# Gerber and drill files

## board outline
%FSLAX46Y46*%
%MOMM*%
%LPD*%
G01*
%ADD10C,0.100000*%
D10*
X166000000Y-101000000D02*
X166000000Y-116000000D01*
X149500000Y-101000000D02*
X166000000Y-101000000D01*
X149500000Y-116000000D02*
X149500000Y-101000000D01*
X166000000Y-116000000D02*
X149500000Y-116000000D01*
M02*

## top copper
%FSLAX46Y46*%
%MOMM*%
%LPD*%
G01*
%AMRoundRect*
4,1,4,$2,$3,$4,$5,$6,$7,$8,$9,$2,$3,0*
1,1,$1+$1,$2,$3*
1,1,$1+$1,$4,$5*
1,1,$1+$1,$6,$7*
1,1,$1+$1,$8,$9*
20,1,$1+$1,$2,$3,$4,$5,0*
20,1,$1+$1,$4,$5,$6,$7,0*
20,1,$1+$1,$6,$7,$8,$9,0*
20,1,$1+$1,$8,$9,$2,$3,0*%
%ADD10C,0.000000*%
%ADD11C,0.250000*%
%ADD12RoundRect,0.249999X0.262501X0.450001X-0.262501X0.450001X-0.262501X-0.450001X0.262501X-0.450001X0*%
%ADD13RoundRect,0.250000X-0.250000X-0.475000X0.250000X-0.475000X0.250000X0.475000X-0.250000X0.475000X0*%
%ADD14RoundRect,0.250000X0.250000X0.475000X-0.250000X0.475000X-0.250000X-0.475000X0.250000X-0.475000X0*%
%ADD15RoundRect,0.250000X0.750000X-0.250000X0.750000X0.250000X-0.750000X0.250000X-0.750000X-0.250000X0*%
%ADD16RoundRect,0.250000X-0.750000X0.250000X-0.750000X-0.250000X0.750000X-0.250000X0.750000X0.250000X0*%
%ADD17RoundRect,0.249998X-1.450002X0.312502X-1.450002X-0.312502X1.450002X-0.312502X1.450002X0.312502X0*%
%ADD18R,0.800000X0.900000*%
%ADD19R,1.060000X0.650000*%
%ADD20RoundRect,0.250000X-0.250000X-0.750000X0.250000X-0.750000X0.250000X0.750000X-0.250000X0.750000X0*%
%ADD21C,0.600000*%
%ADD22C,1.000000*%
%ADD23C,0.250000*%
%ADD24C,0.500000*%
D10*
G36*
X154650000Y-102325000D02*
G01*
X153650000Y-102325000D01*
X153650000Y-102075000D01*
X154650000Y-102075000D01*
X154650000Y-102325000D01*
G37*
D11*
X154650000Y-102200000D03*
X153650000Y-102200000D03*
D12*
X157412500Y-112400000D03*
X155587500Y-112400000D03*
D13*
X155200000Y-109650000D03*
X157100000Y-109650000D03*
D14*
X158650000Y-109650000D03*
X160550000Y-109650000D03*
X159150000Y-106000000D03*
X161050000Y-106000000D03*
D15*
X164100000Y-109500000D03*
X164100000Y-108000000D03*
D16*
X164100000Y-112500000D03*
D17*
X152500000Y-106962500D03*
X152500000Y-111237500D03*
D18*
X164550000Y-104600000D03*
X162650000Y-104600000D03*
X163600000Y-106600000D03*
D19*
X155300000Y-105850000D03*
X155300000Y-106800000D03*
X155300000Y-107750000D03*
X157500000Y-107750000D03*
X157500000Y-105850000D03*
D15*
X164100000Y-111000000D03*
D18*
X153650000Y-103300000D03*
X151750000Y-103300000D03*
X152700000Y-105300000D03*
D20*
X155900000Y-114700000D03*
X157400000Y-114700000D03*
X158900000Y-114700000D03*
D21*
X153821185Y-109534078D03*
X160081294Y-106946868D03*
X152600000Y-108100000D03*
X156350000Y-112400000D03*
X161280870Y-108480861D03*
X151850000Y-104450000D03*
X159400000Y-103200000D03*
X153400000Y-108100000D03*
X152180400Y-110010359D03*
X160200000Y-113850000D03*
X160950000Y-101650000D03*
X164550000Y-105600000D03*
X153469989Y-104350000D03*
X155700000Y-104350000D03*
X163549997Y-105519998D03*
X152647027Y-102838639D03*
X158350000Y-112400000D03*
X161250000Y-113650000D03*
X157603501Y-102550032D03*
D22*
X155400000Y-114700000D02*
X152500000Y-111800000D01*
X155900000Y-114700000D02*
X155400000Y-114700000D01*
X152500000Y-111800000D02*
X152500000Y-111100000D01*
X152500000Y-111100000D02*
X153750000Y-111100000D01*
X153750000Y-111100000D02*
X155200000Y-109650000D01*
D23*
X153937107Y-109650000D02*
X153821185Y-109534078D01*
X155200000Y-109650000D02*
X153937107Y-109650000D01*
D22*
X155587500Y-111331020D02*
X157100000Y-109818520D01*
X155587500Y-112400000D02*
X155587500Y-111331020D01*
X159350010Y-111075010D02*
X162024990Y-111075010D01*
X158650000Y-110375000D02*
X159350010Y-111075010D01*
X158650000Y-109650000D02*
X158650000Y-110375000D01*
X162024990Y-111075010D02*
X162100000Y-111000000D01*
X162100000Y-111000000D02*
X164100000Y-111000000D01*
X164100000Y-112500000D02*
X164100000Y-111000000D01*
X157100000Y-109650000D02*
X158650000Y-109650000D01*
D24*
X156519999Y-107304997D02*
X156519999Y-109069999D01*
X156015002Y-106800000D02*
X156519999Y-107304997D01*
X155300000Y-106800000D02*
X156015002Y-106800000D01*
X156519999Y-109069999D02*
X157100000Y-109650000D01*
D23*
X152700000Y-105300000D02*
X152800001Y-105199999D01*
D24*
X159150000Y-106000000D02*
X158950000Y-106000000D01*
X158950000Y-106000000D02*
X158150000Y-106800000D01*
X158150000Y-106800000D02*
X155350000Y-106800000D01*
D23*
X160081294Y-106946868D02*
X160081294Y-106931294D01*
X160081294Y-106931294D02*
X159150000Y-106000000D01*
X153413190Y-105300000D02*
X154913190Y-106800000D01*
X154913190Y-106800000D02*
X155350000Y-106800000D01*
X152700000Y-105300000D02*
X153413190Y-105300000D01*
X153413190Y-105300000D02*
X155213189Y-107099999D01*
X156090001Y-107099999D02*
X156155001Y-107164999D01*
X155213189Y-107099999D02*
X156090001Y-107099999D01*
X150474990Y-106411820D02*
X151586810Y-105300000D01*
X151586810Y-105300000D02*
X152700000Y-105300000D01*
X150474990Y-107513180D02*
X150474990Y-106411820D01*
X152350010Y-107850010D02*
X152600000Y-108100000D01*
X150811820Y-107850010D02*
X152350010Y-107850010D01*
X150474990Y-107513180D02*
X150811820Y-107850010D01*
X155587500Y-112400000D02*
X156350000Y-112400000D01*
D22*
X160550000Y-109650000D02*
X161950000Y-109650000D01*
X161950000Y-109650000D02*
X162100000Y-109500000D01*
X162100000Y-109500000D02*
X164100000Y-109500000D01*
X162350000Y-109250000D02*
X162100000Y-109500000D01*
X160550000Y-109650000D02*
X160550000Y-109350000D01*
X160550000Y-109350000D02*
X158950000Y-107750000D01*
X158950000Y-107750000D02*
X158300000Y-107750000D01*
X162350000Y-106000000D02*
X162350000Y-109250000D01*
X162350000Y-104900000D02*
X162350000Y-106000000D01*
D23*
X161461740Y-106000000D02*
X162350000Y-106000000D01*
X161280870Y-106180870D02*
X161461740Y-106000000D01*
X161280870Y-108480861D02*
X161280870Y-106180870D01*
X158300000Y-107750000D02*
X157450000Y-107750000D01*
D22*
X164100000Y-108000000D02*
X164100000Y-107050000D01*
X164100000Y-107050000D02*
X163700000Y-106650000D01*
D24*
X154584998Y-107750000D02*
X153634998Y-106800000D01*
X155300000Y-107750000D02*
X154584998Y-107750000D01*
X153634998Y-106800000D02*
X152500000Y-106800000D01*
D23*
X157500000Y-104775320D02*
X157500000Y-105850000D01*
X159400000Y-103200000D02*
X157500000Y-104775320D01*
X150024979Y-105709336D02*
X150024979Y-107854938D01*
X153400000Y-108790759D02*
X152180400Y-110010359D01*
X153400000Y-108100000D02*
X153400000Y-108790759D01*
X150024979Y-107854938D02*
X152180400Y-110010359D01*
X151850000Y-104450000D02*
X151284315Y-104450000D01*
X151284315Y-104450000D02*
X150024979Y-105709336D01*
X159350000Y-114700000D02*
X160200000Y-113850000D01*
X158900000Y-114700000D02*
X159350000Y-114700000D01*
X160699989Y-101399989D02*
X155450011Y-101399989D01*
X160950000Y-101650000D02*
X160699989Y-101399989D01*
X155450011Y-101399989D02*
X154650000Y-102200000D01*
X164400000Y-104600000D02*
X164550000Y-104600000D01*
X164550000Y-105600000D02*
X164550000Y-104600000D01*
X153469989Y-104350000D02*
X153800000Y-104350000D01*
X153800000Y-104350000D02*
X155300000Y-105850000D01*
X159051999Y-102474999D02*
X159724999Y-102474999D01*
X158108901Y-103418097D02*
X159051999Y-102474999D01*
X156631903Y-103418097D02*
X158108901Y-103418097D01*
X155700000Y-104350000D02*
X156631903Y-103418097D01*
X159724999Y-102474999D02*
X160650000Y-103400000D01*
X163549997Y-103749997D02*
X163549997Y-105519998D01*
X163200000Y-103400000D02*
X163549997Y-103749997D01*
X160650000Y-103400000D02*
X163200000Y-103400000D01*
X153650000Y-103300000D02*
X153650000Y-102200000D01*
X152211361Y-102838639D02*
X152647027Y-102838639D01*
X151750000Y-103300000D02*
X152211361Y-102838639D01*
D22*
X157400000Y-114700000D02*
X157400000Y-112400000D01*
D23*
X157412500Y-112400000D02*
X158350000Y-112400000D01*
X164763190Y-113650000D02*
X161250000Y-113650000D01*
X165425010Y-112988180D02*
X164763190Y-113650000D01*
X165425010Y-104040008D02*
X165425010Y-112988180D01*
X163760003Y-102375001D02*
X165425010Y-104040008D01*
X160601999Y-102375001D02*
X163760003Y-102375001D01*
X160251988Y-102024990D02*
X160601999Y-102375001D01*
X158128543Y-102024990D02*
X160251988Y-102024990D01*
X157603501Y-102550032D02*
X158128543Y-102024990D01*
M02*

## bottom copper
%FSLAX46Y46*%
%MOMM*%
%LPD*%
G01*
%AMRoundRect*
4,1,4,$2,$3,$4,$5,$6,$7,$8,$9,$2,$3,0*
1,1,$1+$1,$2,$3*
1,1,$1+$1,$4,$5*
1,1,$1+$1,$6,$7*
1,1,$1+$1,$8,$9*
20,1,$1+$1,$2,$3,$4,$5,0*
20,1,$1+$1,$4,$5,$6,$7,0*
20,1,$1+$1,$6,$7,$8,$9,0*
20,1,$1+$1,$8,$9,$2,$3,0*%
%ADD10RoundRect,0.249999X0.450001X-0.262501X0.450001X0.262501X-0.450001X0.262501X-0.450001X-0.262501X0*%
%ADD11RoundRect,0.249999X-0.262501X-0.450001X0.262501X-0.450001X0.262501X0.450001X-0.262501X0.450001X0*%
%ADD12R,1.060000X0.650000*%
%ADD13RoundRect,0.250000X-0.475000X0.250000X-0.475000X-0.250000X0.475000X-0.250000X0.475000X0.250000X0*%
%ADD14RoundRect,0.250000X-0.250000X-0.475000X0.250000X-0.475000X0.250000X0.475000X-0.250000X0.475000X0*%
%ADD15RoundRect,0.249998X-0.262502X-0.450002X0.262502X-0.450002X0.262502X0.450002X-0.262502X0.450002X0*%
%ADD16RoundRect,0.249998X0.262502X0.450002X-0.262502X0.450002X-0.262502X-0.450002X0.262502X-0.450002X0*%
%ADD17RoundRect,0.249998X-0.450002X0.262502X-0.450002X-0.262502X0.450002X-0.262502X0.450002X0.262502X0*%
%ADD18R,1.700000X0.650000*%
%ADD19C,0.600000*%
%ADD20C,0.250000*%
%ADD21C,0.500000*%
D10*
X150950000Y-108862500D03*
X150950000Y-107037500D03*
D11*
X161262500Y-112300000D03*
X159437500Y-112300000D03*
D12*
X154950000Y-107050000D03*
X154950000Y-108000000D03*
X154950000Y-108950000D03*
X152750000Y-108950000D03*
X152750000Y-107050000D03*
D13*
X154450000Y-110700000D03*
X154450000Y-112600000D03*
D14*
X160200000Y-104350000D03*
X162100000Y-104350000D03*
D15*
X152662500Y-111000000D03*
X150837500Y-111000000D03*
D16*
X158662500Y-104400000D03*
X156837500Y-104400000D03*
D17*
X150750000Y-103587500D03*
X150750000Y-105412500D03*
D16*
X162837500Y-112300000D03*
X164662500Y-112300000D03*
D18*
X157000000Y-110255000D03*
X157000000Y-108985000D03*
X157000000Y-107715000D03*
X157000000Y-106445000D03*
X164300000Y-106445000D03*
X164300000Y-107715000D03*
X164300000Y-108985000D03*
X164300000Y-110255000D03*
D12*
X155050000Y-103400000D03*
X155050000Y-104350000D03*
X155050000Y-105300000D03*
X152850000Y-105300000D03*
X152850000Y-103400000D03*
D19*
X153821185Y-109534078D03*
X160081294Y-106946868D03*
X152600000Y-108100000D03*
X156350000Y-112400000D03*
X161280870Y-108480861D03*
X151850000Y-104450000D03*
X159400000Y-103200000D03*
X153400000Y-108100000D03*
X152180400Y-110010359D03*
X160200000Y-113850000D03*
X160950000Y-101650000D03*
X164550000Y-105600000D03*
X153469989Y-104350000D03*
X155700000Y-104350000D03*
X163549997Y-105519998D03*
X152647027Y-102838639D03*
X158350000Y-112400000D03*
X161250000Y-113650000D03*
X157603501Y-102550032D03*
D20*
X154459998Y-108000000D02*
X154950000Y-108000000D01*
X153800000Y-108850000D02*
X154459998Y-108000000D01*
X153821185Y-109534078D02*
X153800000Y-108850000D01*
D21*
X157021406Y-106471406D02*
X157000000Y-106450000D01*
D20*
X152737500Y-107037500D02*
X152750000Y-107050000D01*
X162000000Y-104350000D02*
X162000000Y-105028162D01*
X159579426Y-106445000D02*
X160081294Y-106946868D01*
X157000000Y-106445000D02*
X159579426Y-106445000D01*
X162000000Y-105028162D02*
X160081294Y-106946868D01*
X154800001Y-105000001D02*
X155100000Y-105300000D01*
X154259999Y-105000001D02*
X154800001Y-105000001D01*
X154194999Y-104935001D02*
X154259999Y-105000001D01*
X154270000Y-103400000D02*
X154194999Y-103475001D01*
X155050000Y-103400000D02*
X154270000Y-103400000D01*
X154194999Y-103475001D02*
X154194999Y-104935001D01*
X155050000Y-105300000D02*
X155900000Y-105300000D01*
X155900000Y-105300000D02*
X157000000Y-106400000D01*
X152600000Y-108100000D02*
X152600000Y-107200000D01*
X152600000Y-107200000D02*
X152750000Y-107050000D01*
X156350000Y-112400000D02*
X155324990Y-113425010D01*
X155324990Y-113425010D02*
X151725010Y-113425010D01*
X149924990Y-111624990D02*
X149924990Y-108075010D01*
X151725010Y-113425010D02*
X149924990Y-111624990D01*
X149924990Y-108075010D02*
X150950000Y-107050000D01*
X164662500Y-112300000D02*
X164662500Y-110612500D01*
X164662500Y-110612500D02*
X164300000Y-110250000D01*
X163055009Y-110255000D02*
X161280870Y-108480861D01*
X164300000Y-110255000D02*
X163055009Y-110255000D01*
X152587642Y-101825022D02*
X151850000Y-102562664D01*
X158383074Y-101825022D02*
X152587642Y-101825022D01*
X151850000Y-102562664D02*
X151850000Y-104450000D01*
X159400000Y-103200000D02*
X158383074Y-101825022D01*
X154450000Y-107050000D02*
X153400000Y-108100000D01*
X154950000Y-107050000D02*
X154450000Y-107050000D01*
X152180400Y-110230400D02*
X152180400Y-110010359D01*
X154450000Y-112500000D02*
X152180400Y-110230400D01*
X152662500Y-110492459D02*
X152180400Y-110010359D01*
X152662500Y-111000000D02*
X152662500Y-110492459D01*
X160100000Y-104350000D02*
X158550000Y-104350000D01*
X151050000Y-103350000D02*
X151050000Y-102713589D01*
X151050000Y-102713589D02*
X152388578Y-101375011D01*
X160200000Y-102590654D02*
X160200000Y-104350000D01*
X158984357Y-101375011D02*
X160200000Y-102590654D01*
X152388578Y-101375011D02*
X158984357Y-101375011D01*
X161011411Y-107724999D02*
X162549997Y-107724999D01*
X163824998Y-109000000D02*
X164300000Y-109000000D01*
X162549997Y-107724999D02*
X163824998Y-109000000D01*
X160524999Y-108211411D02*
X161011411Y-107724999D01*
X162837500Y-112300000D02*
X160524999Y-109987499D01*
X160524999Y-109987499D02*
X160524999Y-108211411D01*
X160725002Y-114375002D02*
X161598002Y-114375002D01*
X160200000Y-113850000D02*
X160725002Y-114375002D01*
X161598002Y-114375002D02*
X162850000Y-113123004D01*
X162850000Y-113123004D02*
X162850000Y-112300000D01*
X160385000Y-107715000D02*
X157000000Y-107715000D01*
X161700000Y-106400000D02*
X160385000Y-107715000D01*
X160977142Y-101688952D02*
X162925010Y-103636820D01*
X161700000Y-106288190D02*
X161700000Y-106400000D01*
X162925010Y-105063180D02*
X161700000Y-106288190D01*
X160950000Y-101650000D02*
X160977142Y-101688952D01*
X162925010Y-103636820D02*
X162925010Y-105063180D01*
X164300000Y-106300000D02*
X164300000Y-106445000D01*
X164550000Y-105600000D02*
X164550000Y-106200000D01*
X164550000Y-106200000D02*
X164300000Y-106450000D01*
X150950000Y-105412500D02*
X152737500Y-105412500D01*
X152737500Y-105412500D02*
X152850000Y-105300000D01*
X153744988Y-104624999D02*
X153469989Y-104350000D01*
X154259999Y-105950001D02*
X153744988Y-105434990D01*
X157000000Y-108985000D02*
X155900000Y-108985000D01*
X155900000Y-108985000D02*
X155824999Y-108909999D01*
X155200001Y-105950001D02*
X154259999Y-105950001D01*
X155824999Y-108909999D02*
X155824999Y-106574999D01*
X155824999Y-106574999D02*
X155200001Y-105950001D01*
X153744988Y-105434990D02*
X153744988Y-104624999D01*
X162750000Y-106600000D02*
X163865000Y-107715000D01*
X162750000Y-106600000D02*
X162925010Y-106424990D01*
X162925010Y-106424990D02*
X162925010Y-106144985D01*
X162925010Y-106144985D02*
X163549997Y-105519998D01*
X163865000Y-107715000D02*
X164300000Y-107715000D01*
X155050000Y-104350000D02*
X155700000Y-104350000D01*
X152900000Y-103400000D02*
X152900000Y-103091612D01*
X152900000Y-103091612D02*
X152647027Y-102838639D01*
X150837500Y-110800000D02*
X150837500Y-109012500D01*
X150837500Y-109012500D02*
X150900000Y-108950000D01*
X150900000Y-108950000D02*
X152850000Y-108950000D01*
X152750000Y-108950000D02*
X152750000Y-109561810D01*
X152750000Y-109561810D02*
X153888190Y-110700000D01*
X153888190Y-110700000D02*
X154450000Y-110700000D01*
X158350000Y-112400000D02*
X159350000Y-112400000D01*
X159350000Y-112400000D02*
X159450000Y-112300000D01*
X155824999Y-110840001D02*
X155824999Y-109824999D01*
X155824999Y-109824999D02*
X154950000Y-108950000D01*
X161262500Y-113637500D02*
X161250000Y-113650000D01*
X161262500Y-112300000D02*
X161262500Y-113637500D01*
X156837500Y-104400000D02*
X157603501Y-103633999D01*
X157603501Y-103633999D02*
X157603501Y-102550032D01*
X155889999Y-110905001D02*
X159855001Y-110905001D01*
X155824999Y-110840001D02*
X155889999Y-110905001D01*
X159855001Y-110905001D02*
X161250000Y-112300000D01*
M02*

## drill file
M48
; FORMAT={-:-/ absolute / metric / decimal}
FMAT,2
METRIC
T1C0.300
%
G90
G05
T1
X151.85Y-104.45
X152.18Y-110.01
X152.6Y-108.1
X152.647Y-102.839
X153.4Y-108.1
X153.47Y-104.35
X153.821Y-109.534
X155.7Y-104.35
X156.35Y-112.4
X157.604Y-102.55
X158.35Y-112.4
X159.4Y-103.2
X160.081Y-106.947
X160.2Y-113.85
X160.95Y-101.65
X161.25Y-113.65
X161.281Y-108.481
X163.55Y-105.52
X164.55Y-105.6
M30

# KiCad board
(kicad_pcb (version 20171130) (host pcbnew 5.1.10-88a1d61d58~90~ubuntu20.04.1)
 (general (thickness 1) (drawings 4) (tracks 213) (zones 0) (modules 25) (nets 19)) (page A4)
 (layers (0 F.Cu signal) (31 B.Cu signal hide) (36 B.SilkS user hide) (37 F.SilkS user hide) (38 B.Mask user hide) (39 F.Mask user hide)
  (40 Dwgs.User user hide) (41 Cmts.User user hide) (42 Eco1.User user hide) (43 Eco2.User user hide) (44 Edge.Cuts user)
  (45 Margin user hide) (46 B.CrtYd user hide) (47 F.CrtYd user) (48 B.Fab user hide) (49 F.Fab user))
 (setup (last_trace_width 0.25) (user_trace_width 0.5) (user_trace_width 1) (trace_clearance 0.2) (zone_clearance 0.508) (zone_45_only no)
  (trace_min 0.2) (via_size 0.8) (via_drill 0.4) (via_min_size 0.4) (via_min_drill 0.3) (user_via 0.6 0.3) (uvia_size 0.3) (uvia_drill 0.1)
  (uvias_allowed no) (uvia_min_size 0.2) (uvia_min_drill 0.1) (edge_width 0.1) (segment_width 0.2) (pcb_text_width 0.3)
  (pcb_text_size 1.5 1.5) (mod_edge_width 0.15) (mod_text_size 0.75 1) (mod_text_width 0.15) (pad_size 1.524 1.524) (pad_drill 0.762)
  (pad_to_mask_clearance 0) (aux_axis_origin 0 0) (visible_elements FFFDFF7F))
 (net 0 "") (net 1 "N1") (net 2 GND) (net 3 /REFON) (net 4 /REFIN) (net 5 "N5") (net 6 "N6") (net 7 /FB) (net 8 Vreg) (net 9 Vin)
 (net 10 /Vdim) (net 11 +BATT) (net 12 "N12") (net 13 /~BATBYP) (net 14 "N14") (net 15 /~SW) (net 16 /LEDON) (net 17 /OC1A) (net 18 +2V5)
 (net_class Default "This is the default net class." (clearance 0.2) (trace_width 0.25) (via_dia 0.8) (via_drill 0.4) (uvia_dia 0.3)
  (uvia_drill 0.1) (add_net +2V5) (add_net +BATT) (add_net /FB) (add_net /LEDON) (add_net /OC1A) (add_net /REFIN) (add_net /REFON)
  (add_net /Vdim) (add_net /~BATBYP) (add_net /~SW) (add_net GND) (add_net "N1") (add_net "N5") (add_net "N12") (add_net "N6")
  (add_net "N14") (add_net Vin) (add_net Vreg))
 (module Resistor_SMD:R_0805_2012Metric (layer B.Cu) (at 150.95 107.95 90)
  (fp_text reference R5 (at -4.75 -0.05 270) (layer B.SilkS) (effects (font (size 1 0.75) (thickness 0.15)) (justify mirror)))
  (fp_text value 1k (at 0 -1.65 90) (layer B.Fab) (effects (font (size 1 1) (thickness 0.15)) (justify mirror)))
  (pad 1 smd roundrect (at -0.9125 0 90) (size 1.025 1.4) (layers B.Cu B.Paste B.Mask) (roundrect_rratio 0.2439014634146341) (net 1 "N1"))
  (pad 2 smd roundrect (at 0.9125 0 90) (size 1.025 1.4) (layers B.Cu B.Paste B.Mask) (roundrect_rratio 0.2439014634146341) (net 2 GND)))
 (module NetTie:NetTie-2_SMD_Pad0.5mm (layer F.Cu) (at 154.15 102.2 180)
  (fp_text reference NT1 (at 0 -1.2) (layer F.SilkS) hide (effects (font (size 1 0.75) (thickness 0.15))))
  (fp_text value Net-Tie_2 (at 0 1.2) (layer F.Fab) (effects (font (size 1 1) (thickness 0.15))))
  (fp_poly (pts (xy -0.5 -0.125) (xy 0.5 -0.125) (xy 0.5 0.125) (xy -0.5 0.125)) (layer F.Cu) (width 0))
  (pad 1 smd circle (at -0.5 0 180) (size 0.25 0.25) (layers F.Cu) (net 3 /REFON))
  (pad 2 smd circle (at 0.5 0 180) (size 0.25 0.25) (layers F.Cu) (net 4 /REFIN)))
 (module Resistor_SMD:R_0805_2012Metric (layer F.Cu) (at 156.5 112.4 180)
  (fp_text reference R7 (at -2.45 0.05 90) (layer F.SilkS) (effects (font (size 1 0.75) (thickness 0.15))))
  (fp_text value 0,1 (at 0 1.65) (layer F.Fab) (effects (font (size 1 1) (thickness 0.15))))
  (pad 1 smd roundrect (at -0.9125 0 180) (size 1.025 1.4) (layers F.Cu F.Paste F.Mask) (roundrect_rratio 0.2439014634146341) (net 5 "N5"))
  (pad 2 smd roundrect (at 0.9125 0 180) (size 1.025 1.4) (layers F.Cu F.Paste F.Mask) (roundrect_rratio 0.2439014634146341) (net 2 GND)))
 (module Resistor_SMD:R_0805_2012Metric (layer B.Cu) (at 160.35 112.3)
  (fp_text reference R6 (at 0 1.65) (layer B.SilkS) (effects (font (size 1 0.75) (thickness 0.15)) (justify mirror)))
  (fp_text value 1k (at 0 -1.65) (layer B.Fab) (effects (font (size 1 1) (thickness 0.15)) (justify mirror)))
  (pad 2 smd roundrect (at 0.9125 0) (size 1.025 1.4) (layers B.Cu B.Paste B.Mask) (roundrect_rratio 0.2439014634146341) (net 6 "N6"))
  (pad 1 smd roundrect (at -0.9125 0) (size 1.025 1.4) (layers B.Cu B.Paste B.Mask) (roundrect_rratio 0.2439014634146341) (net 5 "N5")))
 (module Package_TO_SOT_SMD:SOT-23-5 (layer B.Cu) (at 153.85 108 180)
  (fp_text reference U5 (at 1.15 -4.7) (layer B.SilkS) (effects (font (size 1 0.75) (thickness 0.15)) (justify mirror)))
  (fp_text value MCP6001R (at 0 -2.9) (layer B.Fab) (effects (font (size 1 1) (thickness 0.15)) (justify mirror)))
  (pad 1 smd rect (at -1.1 0.95 180) (size 1.06 0.65) (layers B.Cu B.Paste B.Mask) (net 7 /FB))
  (pad 2 smd rect (at -1.1 0 180) (size 1.06 0.65) (layers B.Cu B.Paste B.Mask) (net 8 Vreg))
  (pad 3 smd rect (at -1.1 -0.95 180) (size 1.06 0.65) (layers B.Cu B.Paste B.Mask) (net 6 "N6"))
  (pad 4 smd rect (at 1.1 -0.95 180) (size 1.06 0.65) (layers B.Cu B.Paste B.Mask) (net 1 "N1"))
  (pad 5 smd rect (at 1.1 0.95 180) (size 1.06 0.65) (layers B.Cu B.Paste B.Mask) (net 2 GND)))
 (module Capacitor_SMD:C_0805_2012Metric (layer F.Cu) (at 156.15 109.65)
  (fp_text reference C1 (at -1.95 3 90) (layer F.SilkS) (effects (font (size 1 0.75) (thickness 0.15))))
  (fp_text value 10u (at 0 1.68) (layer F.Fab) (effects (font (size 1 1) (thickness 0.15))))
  (pad 1 smd roundrect (at -0.95 0) (size 1 1.45) (layers F.Cu F.Paste F.Mask) (roundrect_rratio 0.25) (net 8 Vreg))
  (pad 2 smd roundrect (at 0.95 0) (size 1 1.45) (layers F.Cu F.Paste F.Mask) (roundrect_rratio 0.25) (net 2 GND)))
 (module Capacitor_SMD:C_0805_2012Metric (layer B.Cu) (at 154.45 111.65 270)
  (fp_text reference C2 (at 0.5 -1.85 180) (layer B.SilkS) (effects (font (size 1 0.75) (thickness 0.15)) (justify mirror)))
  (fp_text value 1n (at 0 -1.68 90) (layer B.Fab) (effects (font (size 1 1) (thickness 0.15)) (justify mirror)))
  (pad 1 smd roundrect (at -0.95 0 270) (size 1 1.45) (layers B.Cu B.Paste B.Mask) (roundrect_rratio 0.25) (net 1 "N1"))
  (pad 2 smd roundrect (at 0.95 0 270) (size 1 1.45) (layers B.Cu B.Paste B.Mask) (roundrect_rratio 0.25) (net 7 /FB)))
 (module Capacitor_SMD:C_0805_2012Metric (layer F.Cu) (at 159.6 109.65 180)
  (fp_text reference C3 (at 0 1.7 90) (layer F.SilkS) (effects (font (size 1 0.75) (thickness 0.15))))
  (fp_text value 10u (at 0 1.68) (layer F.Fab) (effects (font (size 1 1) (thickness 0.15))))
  (pad 2 smd roundrect (at 0.95 0 180) (size 1 1.45) (layers F.Cu F.Paste F.Mask) (roundrect_rratio 0.25) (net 2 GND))
  (pad 1 smd roundrect (at -0.95 0 180) (size 1 1.45) (layers F.Cu F.Paste F.Mask) (roundrect_rratio 0.25) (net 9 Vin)))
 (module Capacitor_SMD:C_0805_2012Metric (layer F.Cu) (at 160.1 106 180)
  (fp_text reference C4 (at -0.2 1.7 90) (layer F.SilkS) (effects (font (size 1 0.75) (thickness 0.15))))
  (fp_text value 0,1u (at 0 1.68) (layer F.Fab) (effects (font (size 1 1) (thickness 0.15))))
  (pad 2 smd roundrect (at 0.95 0 180) (size 1 1.45) (layers F.Cu F.Paste F.Mask) (roundrect_rratio 0.25) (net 2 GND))
  (pad 1 smd roundrect (at -0.95 0 180) (size 1 1.45) (layers F.Cu F.Paste F.Mask) (roundrect_rratio 0.25) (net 9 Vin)))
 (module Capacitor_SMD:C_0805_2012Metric (layer B.Cu) (at 161.15 104.35)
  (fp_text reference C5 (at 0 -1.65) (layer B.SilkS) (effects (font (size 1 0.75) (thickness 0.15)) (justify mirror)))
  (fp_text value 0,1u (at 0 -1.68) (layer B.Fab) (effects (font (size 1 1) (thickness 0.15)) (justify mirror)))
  (pad 1 smd roundrect (at -0.95 0) (size 1 1.45) (layers B.Cu B.Paste B.Mask) (roundrect_rratio 0.25) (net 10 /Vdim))
  (pad 2 smd roundrect (at 0.95 0) (size 1 1.45) (layers B.Cu B.Paste B.Mask) (roundrect_rratio 0.25) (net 2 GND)))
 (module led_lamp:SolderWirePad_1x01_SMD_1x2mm (layer F.Cu) (at 164.1 109.5 90)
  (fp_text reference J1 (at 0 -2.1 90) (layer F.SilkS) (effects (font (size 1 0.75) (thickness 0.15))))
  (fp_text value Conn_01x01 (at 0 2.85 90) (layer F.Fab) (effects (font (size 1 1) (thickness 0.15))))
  (pad 1 smd roundrect (at 0 0 90) (size 1 2) (layers F.Cu F.Paste F.Mask) (roundrect_rratio 0.25) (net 9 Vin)))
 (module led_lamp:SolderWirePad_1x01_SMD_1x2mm (layer F.Cu) (at 164.1 108 90)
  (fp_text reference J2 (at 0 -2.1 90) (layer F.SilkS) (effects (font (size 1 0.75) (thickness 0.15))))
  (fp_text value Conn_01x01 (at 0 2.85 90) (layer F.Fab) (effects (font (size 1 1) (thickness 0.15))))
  (pad 1 smd roundrect (at 0 0 90) (size 1 2) (layers F.Cu F.Paste F.Mask) (roundrect_rratio 0.25) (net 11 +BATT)))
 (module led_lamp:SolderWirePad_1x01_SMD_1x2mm (layer F.Cu) (at 164.1 112.5 270)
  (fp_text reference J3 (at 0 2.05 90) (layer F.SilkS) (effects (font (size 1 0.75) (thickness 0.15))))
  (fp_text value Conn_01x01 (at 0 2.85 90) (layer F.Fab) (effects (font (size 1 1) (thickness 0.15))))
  (pad 1 smd roundrect (at 0 0 270) (size 1 2) (layers F.Cu F.Paste F.Mask) (roundrect_rratio 0.25) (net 2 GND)))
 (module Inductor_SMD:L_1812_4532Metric (layer F.Cu) (at 152.5 109.1 270)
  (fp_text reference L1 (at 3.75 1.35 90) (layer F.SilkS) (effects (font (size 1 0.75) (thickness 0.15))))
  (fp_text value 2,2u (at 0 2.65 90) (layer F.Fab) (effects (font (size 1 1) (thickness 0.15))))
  (pad 1 smd roundrect (at -2.1375 0 270) (size 1.125 3.4) (layers F.Cu F.Paste F.Mask) (roundrect_rratio 0.2222204444444444) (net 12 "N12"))
  (pad 2 smd roundrect (at 2.1375 0 270) (size 1.125 3.4) (layers F.Cu F.Paste F.Mask) (roundrect_rratio 0.2222204444444444) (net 8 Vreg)))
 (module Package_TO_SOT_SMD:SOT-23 (layer F.Cu) (at 163.6 105.6 270)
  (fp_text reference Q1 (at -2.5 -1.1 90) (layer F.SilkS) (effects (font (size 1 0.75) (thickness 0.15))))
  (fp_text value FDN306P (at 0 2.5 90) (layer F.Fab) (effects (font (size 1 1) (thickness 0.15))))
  (pad 1 smd rect (at -1 -0.95 270) (size 0.9 0.8) (layers F.Cu F.Paste F.Mask) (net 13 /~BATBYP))
  (pad 2 smd rect (at -1 0.95 270) (size 0.9 0.8) (layers F.Cu F.Paste F.Mask) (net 9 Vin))
  (pad 3 smd rect (at 1 0 270) (size 0.9 0.8) (layers F.Cu F.Paste F.Mask) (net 11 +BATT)))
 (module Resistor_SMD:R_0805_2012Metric (layer B.Cu) (at 151.75 111)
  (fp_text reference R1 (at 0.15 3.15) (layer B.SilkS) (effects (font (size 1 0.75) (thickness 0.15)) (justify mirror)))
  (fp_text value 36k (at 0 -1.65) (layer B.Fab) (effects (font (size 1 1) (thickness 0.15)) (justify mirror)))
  (pad 2 smd roundrect (at 0.9125 0) (size 1.025 1.4) (layers B.Cu B.Paste B.Mask) (roundrect_rratio 0.2439004878048781) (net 7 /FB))
  (pad 1 smd roundrect (at -0.9125 0) (size 1.025 1.4) (layers B.Cu B.Paste B.Mask) (roundrect_rratio 0.2439004878048781) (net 1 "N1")))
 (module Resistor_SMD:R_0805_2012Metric (layer B.Cu) (at 157.75 104.4 180)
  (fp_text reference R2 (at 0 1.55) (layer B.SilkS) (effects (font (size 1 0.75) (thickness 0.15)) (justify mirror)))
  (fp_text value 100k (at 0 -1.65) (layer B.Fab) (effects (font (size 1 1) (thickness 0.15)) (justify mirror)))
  (pad 1 smd roundrect (at -0.9125 0 180) (size 1.025 1.4) (layers B.Cu B.Paste B.Mask) (roundrect_rratio 0.2439004878048781) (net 10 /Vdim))
  (pad 2 smd roundrect (at 0.9125 0 180) (size 1.025 1.4) (layers B.Cu B.Paste B.Mask) (roundrect_rratio 0.2439004878048781) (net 6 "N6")))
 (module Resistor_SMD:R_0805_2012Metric (layer B.Cu) (at 150.75 104.5 270)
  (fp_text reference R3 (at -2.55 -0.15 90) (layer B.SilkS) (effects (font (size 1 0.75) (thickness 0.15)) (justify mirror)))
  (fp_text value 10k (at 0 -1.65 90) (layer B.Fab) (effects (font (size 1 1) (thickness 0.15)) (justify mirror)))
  (pad 1 smd roundrect (at -0.9125 0 270) (size 1.025 1.4) (layers B.Cu B.Paste B.Mask) (roundrect_rratio 0.2439004878048781) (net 10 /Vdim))
  (pad 2 smd roundrect (at 0.9125 0 270) (size 1.025 1.4) (layers B.Cu B.Paste B.Mask) (roundrect_rratio 0.2439004878048781) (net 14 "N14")))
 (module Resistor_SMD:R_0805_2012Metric (layer B.Cu) (at 163.75 112.3 180)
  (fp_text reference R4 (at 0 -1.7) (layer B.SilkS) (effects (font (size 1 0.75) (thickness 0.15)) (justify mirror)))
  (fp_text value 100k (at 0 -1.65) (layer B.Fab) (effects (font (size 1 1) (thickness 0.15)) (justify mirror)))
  (pad 2 smd roundrect (at 0.9125 0 180) (size 1.025 1.4) (layers B.Cu B.Paste B.Mask) (roundrect_rratio 0.2439004878048781) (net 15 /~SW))
  (pad 1 smd roundrect (at -0.9125 0 180) (size 1.025 1.4) (layers B.Cu B.Paste B.Mask) (roundrect_rratio 0.2439004878048781) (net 9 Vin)))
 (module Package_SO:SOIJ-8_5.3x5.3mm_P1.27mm (layer B.Cu) (at 160.65 108.35)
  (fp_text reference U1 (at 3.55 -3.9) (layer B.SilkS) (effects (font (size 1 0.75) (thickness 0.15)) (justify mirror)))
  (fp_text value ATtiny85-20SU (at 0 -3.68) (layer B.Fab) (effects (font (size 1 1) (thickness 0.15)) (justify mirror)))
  (pad 1 smd rect (at -3.65 1.905) (size 1.7 0.65) (layers B.Cu B.Paste B.Mask))
  (pad 2 smd rect (at -3.65 0.635) (size 1.7 0.65) (layers B.Cu B.Paste B.Mask) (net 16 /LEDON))
  (pad 3 smd rect (at -3.65 -0.635) (size 1.7 0.65) (layers B.Cu B.Paste B.Mask) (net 3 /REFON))
  (pad 4 smd rect (at -3.65 -1.905) (size 1.7 0.65) (layers B.Cu B.Paste B.Mask) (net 2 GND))
  (pad 5 smd rect (at 3.65 -1.905) (size 1.7 0.65) (layers B.Cu B.Paste B.Mask) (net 13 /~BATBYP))
  (pad 6 smd rect (at 3.65 -0.635) (size 1.7 0.65) (layers B.Cu B.Paste B.Mask) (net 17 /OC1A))
  (pad 7 smd rect (at 3.65 0.635) (size 1.7 0.65) (layers B.Cu B.Paste B.Mask) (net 15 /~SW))
  (pad 8 smd rect (at 3.65 1.905) (size 1.7 0.65) (layers B.Cu B.Paste B.Mask) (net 9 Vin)))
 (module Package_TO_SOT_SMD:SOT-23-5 (layer F.Cu) (at 156.4 106.8)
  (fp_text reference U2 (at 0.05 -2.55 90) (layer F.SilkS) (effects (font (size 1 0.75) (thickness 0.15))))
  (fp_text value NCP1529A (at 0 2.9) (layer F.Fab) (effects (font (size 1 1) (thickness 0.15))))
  (pad 1 smd rect (at -1.1 -0.95) (size 1.06 0.65) (layers F.Cu F.Paste F.Mask) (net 16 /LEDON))
  (pad 2 smd rect (at -1.1 0) (size 1.06 0.65) (layers F.Cu F.Paste F.Mask) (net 2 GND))
  (pad 3 smd rect (at -1.1 0.95) (size 1.06 0.65) (layers F.Cu F.Paste F.Mask) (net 12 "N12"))
  (pad 4 smd rect (at 1.1 0.95) (size 1.06 0.65) (layers F.Cu F.Paste F.Mask) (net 9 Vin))
  (pad 5 smd rect (at 1.1 -0.95) (size 1.06 0.65) (layers F.Cu F.Paste F.Mask) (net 7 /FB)))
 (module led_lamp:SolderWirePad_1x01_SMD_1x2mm (layer F.Cu) (at 164.1 111 90)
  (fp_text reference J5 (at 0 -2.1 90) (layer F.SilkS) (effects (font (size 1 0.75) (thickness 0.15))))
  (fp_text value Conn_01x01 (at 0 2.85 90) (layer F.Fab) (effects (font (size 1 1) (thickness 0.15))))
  (pad 1 smd roundrect (at 0 0 90) (size 1 2) (layers F.Cu F.Paste F.Mask) (roundrect_rratio 0.25) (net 2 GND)))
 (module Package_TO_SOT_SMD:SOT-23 (layer F.Cu) (at 152.7 104.3 270)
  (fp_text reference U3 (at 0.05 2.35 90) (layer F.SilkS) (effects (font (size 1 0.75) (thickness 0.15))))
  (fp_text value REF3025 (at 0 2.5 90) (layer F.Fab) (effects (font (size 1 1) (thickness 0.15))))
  (pad 1 smd rect (at -1 -0.95 270) (size 0.9 0.8) (layers F.Cu F.Paste F.Mask) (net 4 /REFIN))
  (pad 2 smd rect (at -1 0.95 270) (size 0.9 0.8) (layers F.Cu F.Paste F.Mask) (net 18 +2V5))
  (pad 3 smd rect (at 1 0 270) (size 0.9 0.8) (layers F.Cu F.Paste F.Mask) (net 2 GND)))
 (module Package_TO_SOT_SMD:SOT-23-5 (layer B.Cu) (at 153.95 104.35 180)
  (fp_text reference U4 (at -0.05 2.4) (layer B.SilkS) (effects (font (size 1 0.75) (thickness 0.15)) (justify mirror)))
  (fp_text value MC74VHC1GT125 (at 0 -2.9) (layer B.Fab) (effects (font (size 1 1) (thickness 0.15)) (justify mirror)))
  (pad 1 smd rect (at -1.1 0.95 180) (size 1.06 0.65) (layers B.Cu B.Paste B.Mask) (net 2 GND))
  (pad 2 smd rect (at -1.1 0 180) (size 1.06 0.65) (layers B.Cu B.Paste B.Mask) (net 17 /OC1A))
  (pad 3 smd rect (at -1.1 -0.95 180) (size 1.06 0.65) (layers B.Cu B.Paste B.Mask) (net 2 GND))
  (pad 4 smd rect (at 1.1 -0.95 180) (size 1.06 0.65) (layers B.Cu B.Paste B.Mask) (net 14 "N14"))
  (pad 5 smd rect (at 1.1 0.95 180) (size 1.06 0.65) (layers B.Cu B.Paste B.Mask) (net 18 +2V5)))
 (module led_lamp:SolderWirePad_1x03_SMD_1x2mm (layer F.Cu) (at 155.9 114.7)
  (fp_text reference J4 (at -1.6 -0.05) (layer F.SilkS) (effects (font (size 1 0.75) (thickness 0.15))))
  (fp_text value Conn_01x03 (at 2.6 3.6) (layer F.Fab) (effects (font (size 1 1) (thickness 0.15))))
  (pad 1 smd roundrect (at 0 0) (size 1 2) (layers F.Cu F.Paste F.Mask) (roundrect_rratio 0.25) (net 8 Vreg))
  (pad 2 smd roundrect (at 1.5 0) (size 1 2) (layers F.Cu F.Paste F.Mask) (roundrect_rratio 0.25) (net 5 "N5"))
  (pad 3 smd roundrect (at 3 0) (size 1 2) (layers F.Cu F.Paste F.Mask) (roundrect_rratio 0.25) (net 15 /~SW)))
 (gr_line (start 166 101) (end 166 116) (layer Edge.Cuts) (width 0.1))
 (gr_line (start 149.5 101) (end 166 101) (layer Edge.Cuts) (width 0.1))
 (gr_line (start 149.5 116) (end 149.5 101) (layer Edge.Cuts) (width 0.1))
 (gr_line (start 166 116) (end 149.5 116) (layer Edge.Cuts) (width 0.1))
 (segment (start 155.4 114.7) (end 152.5 111.8) (width 1) (layer F.Cu) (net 8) (status 10))
 (segment (start 155.9 114.7) (end 155.4 114.7) (width 1) (layer F.Cu) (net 8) (status 30))
 (segment (start 152.5 111.8) (end 152.5 111.1) (width 1) (layer F.Cu) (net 8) (status 20))
 (segment (start 152.5 111.1) (end 153.75 111.1) (width 1) (layer F.Cu) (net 8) (status 30))
 (segment (start 153.75 111.1) (end 155.2 109.65) (width 1) (layer F.Cu) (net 8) (status 30))
 (via (at 153.821185 109.534078) (size 0.6) (drill 0.3) (layers F.Cu B.Cu) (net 8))
 (segment (start 153.937107 109.65) (end 153.821185 109.534078) (width 0.25) (layer F.Cu) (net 8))
 (segment (start 155.2 109.65) (end 153.937107 109.65) (width 0.25) (layer F.Cu) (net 8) (status 10))
 (segment (start 154.459998 108) (end 154.95 108) (width 0.25) (layer B.Cu) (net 8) (status 30))
 (segment (start 153.8 108.85) (end 154.459998 108) (width 0.25) (layer B.Cu) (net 8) (status 20))
 (segment (start 153.821185 109.534078) (end 153.8 108.85) (width 0.25) (layer B.Cu) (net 8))
 (segment (start 155.5875 111.33102) (end 157.1 109.81852) (width 1) (layer F.Cu) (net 2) (status 20))
 (segment (start 155.5875 112.4) (end 155.5875 111.33102) (width 1) (layer F.Cu) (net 2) (status 10))
 (segment (start 159.35001 111.07501) (end 162.02499 111.07501) (width 1) (layer F.Cu) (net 2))
 (segment (start 158.65 110.375) (end 159.35001 111.07501) (width 1) (layer F.Cu) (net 2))
 (segment (start 158.65 109.65) (end 158.65 110.375) (width 1) (layer F.Cu) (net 2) (status 10))
 (segment (start 162.02499 111.07501) (end 162.1 111) (width 1) (layer F.Cu) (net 2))
 (segment (start 162.1 111) (end 164.1 111) (width 1) (layer F.Cu) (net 2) (status 20))
 (segment (start 164.1 112.5) (end 164.1 111) (width 1) (layer F.Cu) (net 2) (status 30))
 (segment (start 157.1 109.65) (end 158.65 109.65) (width 1) (layer F.Cu) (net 2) (status 30))
 (segment (start 156.519999 107.304997) (end 156.519999 109.069999) (width 0.5) (layer F.Cu) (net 2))
 (segment (start 156.015002 106.8) (end 156.519999 107.304997) (width 0.5) (layer F.Cu) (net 2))
 (segment (start 155.3 106.8) (end 156.015002 106.8) (width 0.5) (layer F.Cu) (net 2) (status 10))
 (segment (start 156.519999 109.069999) (end 157.1 109.65) (width 0.5) (layer F.Cu) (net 2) (status 20))
 (segment (start 152.7 105.3) (end 152.800001 105.199999) (width 0.25) (layer F.Cu) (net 2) (status 30))
 (segment (start 157.021406 106.471406) (end 157 106.45) (width 0.5) (layer B.Cu) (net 2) (status 30))
 (segment (start 159.15 106) (end 158.95 106) (width 0.5) (layer F.Cu) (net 2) (status 30))
 (segment (start 158.95 106) (end 158.15 106.8) (width 0.5) (layer F.Cu) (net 2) (status 10))
 (segment (start 158.15 106.8) (end 155.35 106.8) (width 0.5) (layer F.Cu) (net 2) (status 20))
 (segment (start 152.7375 107.0375) (end 152.75 107.05) (width 0.25) (layer B.Cu) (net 2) (status 30))
 (segment (start 162 104.35) (end 162 105.028162) (width 0.25) (layer B.Cu) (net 2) (status 30))
 (via (at 160.081294 106.946868) (size 0.6) (drill 0.3) (layers F.Cu B.Cu) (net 2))
 (segment (start 159.579426 106.445) (end 160.081294 106.946868) (width 0.25) (layer B.Cu) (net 2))
 (segment (start 157 106.445) (end 159.579426 106.445) (width 0.25) (layer B.Cu) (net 2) (status 10))
 (segment (start 162 105.028162) (end 160.081294 106.946868) (width 0.25) (layer B.Cu) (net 2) (status 10))
 (segment (start 160.081294 106.946868) (end 160.081294 106.931294) (width 0.25) (layer F.Cu) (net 2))
 (segment (start 160.081294 106.931294) (end 159.15 106) (width 0.25) (layer F.Cu) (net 2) (status 20))
 (segment (start 154.800001 105.000001) (end 155.1 105.3) (width 0.25) (layer B.Cu) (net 2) (status 30))
 (segment (start 154.259999 105.000001) (end 154.800001 105.000001) (width 0.25) (layer B.Cu) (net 2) (status 20))
 (segment (start 154.194999 104.935001) (end 154.259999 105.000001) (width 0.25) (layer B.Cu) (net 2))
 (segment (start 154.27 103.4) (end 154.194999 103.475001) (width 0.25) (layer B.Cu) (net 2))
 (segment (start 155.05 103.4) (end 154.27 103.4) (width 0.25) (layer B.Cu) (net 2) (status 10))
 (segment (start 154.194999 103.475001) (end 154.194999 104.935001) (width 0.25) (layer B.Cu) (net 2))
 (segment (start 153.41319 105.3) (end 154.91319 106.8) (width 0.25) (layer F.Cu) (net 2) (status 20))
 (segment (start 154.91319 106.8) (end 155.35 106.8) (width 0.25) (layer F.Cu) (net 2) (status 30))
 (segment (start 155.05 105.3) (end 155.9 105.3) (width 0.25) (layer B.Cu) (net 2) (status 10))
 (segment (start 155.9 105.3) (end 157 106.4) (width 0.25) (layer B.Cu) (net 2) (status 20))
 (segment (start 152.7 105.3) (end 153.41319 105.3) (width 0.25) (layer F.Cu) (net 2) (status 10))
 (segment (start 153.41319 105.3) (end 155.213189 107.099999) (width 0.25) (layer F.Cu) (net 2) (status 20))
 (segment (start 156.090001 107.099999) (end 156.155001 107.164999) (width 0.25) (layer F.Cu) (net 2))
 (segment (start 155.213189 107.099999) (end 156.090001 107.099999) (width 0.25) (layer F.Cu) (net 2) (status 10))
 (via (at 152.6 108.1) (size 0.6) (drill 0.3) (layers F.Cu B.Cu) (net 2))
 (segment (start 150.47499 106.41182) (end 151.58681 105.3) (width 0.25) (layer F.Cu) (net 2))
 (segment (start 151.58681 105.3) (end 152.7 105.3) (width 0.25) (layer F.Cu) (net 2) (status 20))
 (segment (start 150.47499 107.51318) (end 150.47499 106.41182) (width 0.25) (layer F.Cu) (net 2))
 (segment (start 152.6 108.1) (end 152.6 107.2) (width 0.25) (layer B.Cu) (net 2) (status 20))
 (segment (start 152.6 107.2) (end 152.75 107.05) (width 0.25) (layer B.Cu) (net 2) (status 30))
 (segment (start 152.35001 107.85001) (end 152.6 108.1) (width 0.25) (layer F.Cu) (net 2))
 (segment (start 150.81182 107.85001) (end 152.35001 107.85001) (width 0.25) (layer F.Cu) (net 2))
 (segment (start 150.47499 107.51318) (end 150.81182 107.85001) (width 0.25) (layer F.Cu) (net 2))
 (via (at 156.35 112.4) (size 0.6) (drill 0.3) (layers F.Cu B.Cu) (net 2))
 (segment (start 155.5875 112.4) (end 156.35 112.4) (width 0.25) (layer F.Cu) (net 2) (status 10))
 (segment (start 156.35 112.4) (end 155.32499 113.42501) (width 0.25) (layer B.Cu) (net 2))
 (segment (start 155.32499 113.42501) (end 151.72501 113.42501) (width 0.25) (layer B.Cu) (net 2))
 (segment (start 149.92499 111.62499) (end 149.92499 108.07501) (width 0.25) (layer B.Cu) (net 2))
 (segment (start 151.72501 113.42501) (end 149.92499 111.62499) (width 0.25) (layer B.Cu) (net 2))
 (segment (start 149.92499 108.07501) (end 150.95 107.05) (width 0.25) (layer B.Cu) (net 2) (status 20))
 (segment (start 160.55 109.65) (end 161.95 109.65) (width 1) (layer F.Cu) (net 9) (status 10))
 (segment (start 161.95 109.65) (end 162.1 109.5) (width 1) (layer F.Cu) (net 9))
 (segment (start 162.1 109.5) (end 164.1 109.5) (width 1) (layer F.Cu) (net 9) (status 20))
 (segment (start 162.35 109.25) (end 162.1 109.5) (width 1) (layer F.Cu) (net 9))
 (segment (start 160.55 109.65) (end 160.55 109.35) (width 1) (layer F.Cu) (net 9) (status 30))
 (segment (start 160.55 109.35) (end 158.95 107.75) (width 1) (layer F.Cu) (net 9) (status 10))
 (segment (start 158.95 107.75) (end 158.3 107.75) (width 1) (layer F.Cu) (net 9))
 (segment (start 162.35 106) (end 162.35 109.25) (width 1) (layer F.Cu) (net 9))
 (segment (start 162.35 104.9) (end 162.35 106) (width 1) (layer F.Cu) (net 9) (status 10))
 (segment (start 164.6625 112.3) (end 164.6625 110.6125) (width 0.25) (layer B.Cu) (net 9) (status 10))
 (segment (start 164.6625 110.6125) (end 164.3 110.25) (width 0.25) (layer B.Cu) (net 9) (status 20))
 (via (at 161.28087 108.480861) (size 0.6) (drill 0.3) (layers F.Cu B.Cu) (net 9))
 (segment (start 163.055009 110.255) (end 161.28087 108.480861) (width 0.25) (layer B.Cu) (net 9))
 (segment (start 164.3 110.255) (end 163.055009 110.255) (width 0.25) (layer B.Cu) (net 9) (status 10))
 (segment (start 161.46174 106) (end 162.35 106) (width 0.25) (layer F.Cu) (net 9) (status 10))
 (segment (start 161.28087 106.18087) (end 161.46174 106) (width 0.25) (layer F.Cu) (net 9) (status 30))
 (segment (start 161.28087 108.480861) (end 161.28087 106.18087) (width 0.25) (layer F.Cu) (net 9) (status 20))
 (segment (start 158.3 107.75) (end 157.45 107.75) (width 0.25) (layer F.Cu) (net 9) (status 20))
 (segment (start 164.1 108) (end 164.1 107.05) (width 1) (layer F.Cu) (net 11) (status 10))
 (segment (start 164.1 107.05) (end 163.7 106.65) (width 1) (layer F.Cu) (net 11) (status 20))
 (segment (start 154.584998 107.75) (end 153.634998 106.8) (width 0.5) (layer F.Cu) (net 12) (status 20))
 (segment (start 155.3 107.75) (end 154.584998 107.75) (width 0.5) (layer F.Cu) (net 12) (status 10))
 (segment (start 153.634998 106.8) (end 152.5 106.8) (width 0.5) (layer F.Cu) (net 12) (status 30))
 (via (at 151.85 104.45) (size 0.6) (drill 0.3) (layers F.Cu B.Cu) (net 7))
 (segment (start 152.587642 101.825022) (end 151.85 102.562664) (width 0.25) (layer B.Cu) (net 7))
 (segment (start 158.383074 101.825022) (end 152.587642 101.825022) (width 0.25) (layer B.Cu) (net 7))
 (segment (start 157.5 104.77532) (end 157.5 105.85) (width 0.25) (layer F.Cu) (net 7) (status 20))
 (segment (start 151.85 102.562664) (end 151.85 104.45) (width 0.25) (layer B.Cu) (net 7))
 (segment (start 159.4 103.2) (end 157.5 104.77532) (width 0.25) (layer F.Cu) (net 7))
 (segment (start 159.4 103.2) (end 158.383074 101.825022) (width 0.25) (layer B.Cu) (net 7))
 (via (at 159.4 103.2) (size 0.6) (drill 0.3) (layers F.Cu B.Cu) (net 7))
 (via (at 153.4 108.1) (size 0.6) (drill 0.3) (layers F.Cu B.Cu) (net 7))
 (segment (start 154.45 107.05) (end 153.4 108.1) (width 0.25) (layer B.Cu) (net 7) (status 10))
 (segment (start 154.95 107.05) (end 154.45 107.05) (width 0.25) (layer B.Cu) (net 7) (status 30))
 (segment (start 150.024979 105.709336) (end 150.024979 107.854938) (width 0.25) (layer F.Cu) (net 7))
 (via (at 152.1804 110.010359) (size 0.6) (drill 0.3) (layers F.Cu B.Cu) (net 7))
 (segment (start 153.4 108.790759) (end 152.1804 110.010359) (width 0.25) (layer F.Cu) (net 7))
 (segment (start 152.1804 110.2304) (end 152.1804 110.010359) (width 0.25) (layer B.Cu) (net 7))
 (segment (start 154.45 112.5) (end 152.1804 110.2304) (width 0.25) (layer B.Cu) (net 7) (status 10))
 (segment (start 153.4 108.1) (end 153.4 108.790759) (width 0.25) (layer F.Cu) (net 7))
 (segment (start 150.024979 107.854938) (end 152.1804 110.010359) (width 0.25) (layer F.Cu) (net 7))
 (segment (start 151.85 104.45) (end 151.284315 104.45) (width 0.25) (layer F.Cu) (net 7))
 (segment (start 151.284315 104.45) (end 150.024979 105.709336) (width 0.25) (layer F.Cu) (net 7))
 (segment (start 152.6625 110.492459) (end 152.1804 110.010359) (width 0.25) (layer B.Cu) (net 7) (status 10))
 (segment (start 152.6625 111) (end 152.6625 110.492459) (width 0.25) (layer B.Cu) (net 7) (status 30))
 (segment (start 160.1 104.35) (end 158.55 104.35) (width 0.25) (layer B.Cu) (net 10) (status 30))
 (segment (start 151.05 103.35) (end 151.05 102.713589) (width 0.25) (layer B.Cu) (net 10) (status 10))
 (segment (start 151.05 102.713589) (end 152.388578 101.375011) (width 0.25) (layer B.Cu) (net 10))
 (segment (start 160.2 102.590654) (end 160.2 104.35) (width 0.25) (layer B.Cu) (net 10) (status 20))
 (segment (start 158.984357 101.375011) (end 160.2 102.590654) (width 0.25) (layer B.Cu) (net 10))
 (segment (start 152.388578 101.375011) (end 158.984357 101.375011) (width 0.25) (layer B.Cu) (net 10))
 (segment (start 159.35 114.7) (end 160.2 113.85) (width 0.25) (layer F.Cu) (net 15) (status 10))
 (via (at 160.2 113.85) (size 0.6) (drill 0.3) (layers F.Cu B.Cu) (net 15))
 (segment (start 158.9 114.7) (end 159.35 114.7) (width 0.25) (layer F.Cu) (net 15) (status 30))
 (segment (start 161.011411 107.724999) (end 162.549997 107.724999) (width 0.25) (layer B.Cu) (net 15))
 (segment (start 163.824998 109) (end 164.3 109) (width 0.25) (layer B.Cu) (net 15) (status 30))
 (segment (start 162.549997 107.724999) (end 163.824998 109) (width 0.25) (layer B.Cu) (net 15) (status 20))
 (segment (start 160.524999 108.211411) (end 161.011411 107.724999) (width 0.25) (layer B.Cu) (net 15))
 (segment (start 162.8375 112.3) (end 160.524999 109.987499) (width 0.25) (layer B.Cu) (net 15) (status 10))
 (segment (start 160.524999 109.987499) (end 160.524999 108.211411) (width 0.25) (layer B.Cu) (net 15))
 (segment (start 160.725002 114.375002) (end 161.598002 114.375002) (width 0.25) (layer B.Cu) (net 15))
 (segment (start 160.2 113.85) (end 160.725002 114.375002) (width 0.25) (layer B.Cu) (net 15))
 (segment (start 161.598002 114.375002) (end 162.85 113.123004) (width 0.25) (layer B.Cu) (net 15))
 (segment (start 162.85 113.123004) (end 162.85 112.3) (width 0.25) (layer B.Cu) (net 15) (status 20))
 (segment (start 160.385 107.715) (end 157 107.715) (width 0.25) (layer B.Cu) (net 3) (status 20))
 (segment (start 161.7 106.4) (end 160.385 107.715) (width 0.25) (layer B.Cu) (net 3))
 (segment (start 160.977142 101.688952) (end 162.92501 103.63682) (width 0.25) (layer B.Cu) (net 3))
 (segment (start 161.7 106.28819) (end 161.7 106.4) (width 0.25) (layer B.Cu) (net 3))
 (segment (start 162.92501 105.06318) (end 161.7 106.28819) (width 0.25) (layer B.Cu) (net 3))
 (segment (start 160.95 101.65) (end 160.977142 101.688952) (width 0.25) (layer B.Cu) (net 3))
 (segment (start 162.92501 103.63682) (end 162.92501 105.06318) (width 0.25) (layer B.Cu) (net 3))
 (via (at 160.95 101.65) (size 0.6) (drill 0.3) (layers F.Cu B.Cu) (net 3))
 (segment (start 160.699989 101.399989) (end 155.450011 101.399989) (width 0.25) (layer F.Cu) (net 3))
 (segment (start 160.95 101.65) (end 160.699989 101.399989) (width 0.25) (layer F.Cu) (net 3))
 (segment (start 155.450011 101.399989) (end 154.65 102.2) (width 0.25) (layer F.Cu) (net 3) (status 20))
 (segment (start 164.4 104.6) (end 164.55 104.6) (width 0.25) (layer F.Cu) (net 13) (status 30))
 (segment (start 164.3 106.3) (end 164.3 106.445) (width 0.25) (layer B.Cu) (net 13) (status 30))
 (via (at 164.55 105.6) (size 0.6) (drill 0.3) (layers F.Cu B.Cu) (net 13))
 (segment (start 164.55 105.6) (end 164.55 106.2) (width 0.25) (layer B.Cu) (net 13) (status 20))
 (segment (start 164.55 106.2) (end 164.3 106.45) (width 0.25) (layer B.Cu) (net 13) (status 30))
 (segment (start 164.55 105.6) (end 164.55 104.6) (width 0.25) (layer F.Cu) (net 13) (status 20))
 (segment (start 150.95 105.4125) (end 152.7375 105.4125) (width 0.25) (layer B.Cu) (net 14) (status 30))
 (segment (start 152.7375 105.4125) (end 152.85 105.3) (width 0.25) (layer B.Cu) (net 14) (status 30))
 (segment (start 153.744988 104.624999) (end 153.469989 104.35) (width 0.25) (layer B.Cu) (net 16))
 (segment (start 154.259999 105.950001) (end 153.744988 105.43499) (width 0.25) (layer B.Cu) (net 16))
 (segment (start 157 108.985) (end 155.9 108.985) (width 0.25) (layer B.Cu) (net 16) (status 10))
 (via (at 153.469989 104.35) (size 0.6) (drill 0.3) (layers F.Cu B.Cu) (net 16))
 (segment (start 155.9 108.985) (end 155.824999 108.909999) (width 0.25) (layer B.Cu) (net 16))
 (segment (start 155.200001 105.950001) (end 154.259999 105.950001) (width 0.25) (layer B.Cu) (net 16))
 (segment (start 155.824999 108.909999) (end 155.824999 106.574999) (width 0.25) (layer B.Cu) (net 16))
 (segment (start 155.824999 106.574999) (end 155.200001 105.950001) (width 0.25) (layer B.Cu) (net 16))
 (segment (start 153.744988 105.43499) (end 153.744988 104.624999) (width 0.25) (layer B.Cu) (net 16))
 (segment (start 153.469989 104.35) (end 153.8 104.35) (width 0.25) (layer F.Cu) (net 16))
 (segment (start 153.8 104.35) (end 155.3 105.85) (width 0.25) (layer F.Cu) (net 16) (status 20))
 (via (at 155.7 104.35) (size 0.6) (drill 0.3) (layers F.Cu B.Cu) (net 17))
 (segment (start 162.75 106.6) (end 163.865 107.715) (width 0.25) (layer B.Cu) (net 17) (status 20))
 (segment (start 162.75 106.6) (end 162.92501 106.42499) (width 0.25) (layer B.Cu) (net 17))
 (segment (start 162.92501 106.42499) (end 162.92501 106.144985) (width 0.25) (layer B.Cu) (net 17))
 (segment (start 162.92501 106.144985) (end 163.549997 105.519998) (width 0.25) (layer B.Cu) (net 17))
 (via (at 163.549997 105.519998) (size 0.6) (drill 0.3) (layers F.Cu B.Cu) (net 17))
 (segment (start 163.865 107.715) (end 164.3 107.715) (width 0.25) (layer B.Cu) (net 17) (status 30))
 (segment (start 155.05 104.35) (end 155.7 104.35) (width 0.25) (layer B.Cu) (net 17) (status 10))
 (segment (start 159.051999 102.474999) (end 159.724999 102.474999) (width 0.25) (layer F.Cu) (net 17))
 (segment (start 158.108901 103.418097) (end 159.051999 102.474999) (width 0.25) (layer F.Cu) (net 17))
 (segment (start 156.631903 103.418097) (end 158.108901 103.418097) (width 0.25) (layer F.Cu) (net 17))
 (segment (start 155.7 104.35) (end 156.631903 103.418097) (width 0.25) (layer F.Cu) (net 17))
 (segment (start 159.724999 102.474999) (end 160.65 103.4) (width 0.25) (layer F.Cu) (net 17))
 (segment (start 163.549997 103.749997) (end 163.549997 105.519998) (width 0.25) (layer F.Cu) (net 17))
 (segment (start 163.2 103.4) (end 163.549997 103.749997) (width 0.25) (layer F.Cu) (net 17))
 (segment (start 160.65 103.4) (end 163.2 103.4) (width 0.25) (layer F.Cu) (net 17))
 (segment (start 153.65 103.3) (end 153.65 102.2) (width 0.25) (layer F.Cu) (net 4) (status 30))
 (segment (start 152.211361 102.838639) (end 152.647027 102.838639) (width 0.25) (layer F.Cu) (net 18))
 (segment (start 152.9 103.4) (end 152.9 103.091612) (width 0.25) (layer B.Cu) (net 18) (status 30))
 (via (at 152.647027 102.838639) (size 0.6) (drill 0.3) (layers F.Cu B.Cu) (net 18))
 (segment (start 152.9 103.091612) (end 152.647027 102.838639) (width 0.25) (layer B.Cu) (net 18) (status 10))
 (segment (start 151.75 103.3) (end 152.211361 102.838639) (width 0.25) (layer F.Cu) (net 18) (status 10))
 (segment (start 150.8375 110.8) (end 150.8375 109.0125) (width 0.25) (layer B.Cu) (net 1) (status 30))
 (segment (start 150.8375 109.0125) (end 150.9 108.95) (width 0.25) (layer B.Cu) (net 1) (status 30))
 (segment (start 150.9 108.95) (end 152.85 108.95) (width 0.25) (layer B.Cu) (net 1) (status 30))
 (segment (start 152.75 108.95) (end 152.75 109.56181) (width 0.25) (layer B.Cu) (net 1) (status 10))
 (segment (start 152.75 109.56181) (end 153.88819 110.7) (width 0.25) (layer B.Cu) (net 1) (status 20))
 (segment (start 153.88819 110.7) (end 154.45 110.7) (width 0.25) (layer B.Cu) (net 1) (status 30))
 (segment (start 157.4 114.7) (end 157.4 112.4) (width 1) (layer F.Cu) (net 5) (status 30))
 (segment (start 157.4125 112.4) (end 158.35 112.4) (width 0.25) (layer F.Cu) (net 5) (status 10))
 (via (at 158.35 112.4) (size 0.6) (drill 0.3) (layers F.Cu B.Cu) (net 5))
 (segment (start 158.35 112.4) (end 159.35 112.4) (width 0.25) (layer B.Cu) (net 5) (status 20))
 (segment (start 159.35 112.4) (end 159.45 112.3) (width 0.25) (layer B.Cu) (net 5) (status 30))
 (segment (start 155.824999 110.840001) (end 155.824999 109.824999) (width 0.25) (layer B.Cu) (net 6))
 (segment (start 155.824999 109.824999) (end 154.95 108.95) (width 0.25) (layer B.Cu) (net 6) (status 20))
 (via (at 161.25 113.65) (size 0.6) (drill 0.3) (layers F.Cu B.Cu) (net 6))
 (segment (start 161.2625 113.6375) (end 161.25 113.65) (width 0.25) (layer B.Cu) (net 6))
 (segment (start 161.2625 112.3) (end 161.2625 113.6375) (width 0.25) (layer B.Cu) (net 6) (status 10))
 (via (at 157.603501 102.550032) (size 0.6) (drill 0.3) (layers F.Cu B.Cu) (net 6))
 (segment (start 156.8375 104.4) (end 157.603501 103.633999) (width 0.25) (layer B.Cu) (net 6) (status 10))
 (segment (start 157.603501 103.633999) (end 157.603501 102.550032) (width 0.25) (layer B.Cu) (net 6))
 (segment (start 164.76319 113.65) (end 161.25 113.65) (width 0.25) (layer F.Cu) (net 6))
 (segment (start 165.42501 112.98818) (end 164.76319 113.65) (width 0.25) (layer F.Cu) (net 6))
 (segment (start 165.42501 104.040008) (end 165.42501 112.98818) (width 0.25) (layer F.Cu) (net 6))
 (segment (start 163.760003 102.375001) (end 165.42501 104.040008) (width 0.25) (layer F.Cu) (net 6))
 (segment (start 160.601999 102.375001) (end 163.760003 102.375001) (width 0.25) (layer F.Cu) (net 6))
 (segment (start 160.251988 102.02499) (end 160.601999 102.375001) (width 0.25) (layer F.Cu) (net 6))
 (segment (start 158.128543 102.02499) (end 160.251988 102.02499) (width 0.25) (layer F.Cu) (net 6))
 (segment (start 157.603501 102.550032) (end 158.128543 102.02499) (width 0.25) (layer F.Cu) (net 6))
 (segment (start 155.889999 110.905001) (end 159.855001 110.905001) (width 0.25) (layer B.Cu) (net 6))
 (segment (start 155.824999 110.840001) (end 155.889999 110.905001) (width 0.25) (layer B.Cu) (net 6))
 (segment (start 159.855001 110.905001) (end 161.25 112.3) (width 0.25) (layer B.Cu) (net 6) (status 20)))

